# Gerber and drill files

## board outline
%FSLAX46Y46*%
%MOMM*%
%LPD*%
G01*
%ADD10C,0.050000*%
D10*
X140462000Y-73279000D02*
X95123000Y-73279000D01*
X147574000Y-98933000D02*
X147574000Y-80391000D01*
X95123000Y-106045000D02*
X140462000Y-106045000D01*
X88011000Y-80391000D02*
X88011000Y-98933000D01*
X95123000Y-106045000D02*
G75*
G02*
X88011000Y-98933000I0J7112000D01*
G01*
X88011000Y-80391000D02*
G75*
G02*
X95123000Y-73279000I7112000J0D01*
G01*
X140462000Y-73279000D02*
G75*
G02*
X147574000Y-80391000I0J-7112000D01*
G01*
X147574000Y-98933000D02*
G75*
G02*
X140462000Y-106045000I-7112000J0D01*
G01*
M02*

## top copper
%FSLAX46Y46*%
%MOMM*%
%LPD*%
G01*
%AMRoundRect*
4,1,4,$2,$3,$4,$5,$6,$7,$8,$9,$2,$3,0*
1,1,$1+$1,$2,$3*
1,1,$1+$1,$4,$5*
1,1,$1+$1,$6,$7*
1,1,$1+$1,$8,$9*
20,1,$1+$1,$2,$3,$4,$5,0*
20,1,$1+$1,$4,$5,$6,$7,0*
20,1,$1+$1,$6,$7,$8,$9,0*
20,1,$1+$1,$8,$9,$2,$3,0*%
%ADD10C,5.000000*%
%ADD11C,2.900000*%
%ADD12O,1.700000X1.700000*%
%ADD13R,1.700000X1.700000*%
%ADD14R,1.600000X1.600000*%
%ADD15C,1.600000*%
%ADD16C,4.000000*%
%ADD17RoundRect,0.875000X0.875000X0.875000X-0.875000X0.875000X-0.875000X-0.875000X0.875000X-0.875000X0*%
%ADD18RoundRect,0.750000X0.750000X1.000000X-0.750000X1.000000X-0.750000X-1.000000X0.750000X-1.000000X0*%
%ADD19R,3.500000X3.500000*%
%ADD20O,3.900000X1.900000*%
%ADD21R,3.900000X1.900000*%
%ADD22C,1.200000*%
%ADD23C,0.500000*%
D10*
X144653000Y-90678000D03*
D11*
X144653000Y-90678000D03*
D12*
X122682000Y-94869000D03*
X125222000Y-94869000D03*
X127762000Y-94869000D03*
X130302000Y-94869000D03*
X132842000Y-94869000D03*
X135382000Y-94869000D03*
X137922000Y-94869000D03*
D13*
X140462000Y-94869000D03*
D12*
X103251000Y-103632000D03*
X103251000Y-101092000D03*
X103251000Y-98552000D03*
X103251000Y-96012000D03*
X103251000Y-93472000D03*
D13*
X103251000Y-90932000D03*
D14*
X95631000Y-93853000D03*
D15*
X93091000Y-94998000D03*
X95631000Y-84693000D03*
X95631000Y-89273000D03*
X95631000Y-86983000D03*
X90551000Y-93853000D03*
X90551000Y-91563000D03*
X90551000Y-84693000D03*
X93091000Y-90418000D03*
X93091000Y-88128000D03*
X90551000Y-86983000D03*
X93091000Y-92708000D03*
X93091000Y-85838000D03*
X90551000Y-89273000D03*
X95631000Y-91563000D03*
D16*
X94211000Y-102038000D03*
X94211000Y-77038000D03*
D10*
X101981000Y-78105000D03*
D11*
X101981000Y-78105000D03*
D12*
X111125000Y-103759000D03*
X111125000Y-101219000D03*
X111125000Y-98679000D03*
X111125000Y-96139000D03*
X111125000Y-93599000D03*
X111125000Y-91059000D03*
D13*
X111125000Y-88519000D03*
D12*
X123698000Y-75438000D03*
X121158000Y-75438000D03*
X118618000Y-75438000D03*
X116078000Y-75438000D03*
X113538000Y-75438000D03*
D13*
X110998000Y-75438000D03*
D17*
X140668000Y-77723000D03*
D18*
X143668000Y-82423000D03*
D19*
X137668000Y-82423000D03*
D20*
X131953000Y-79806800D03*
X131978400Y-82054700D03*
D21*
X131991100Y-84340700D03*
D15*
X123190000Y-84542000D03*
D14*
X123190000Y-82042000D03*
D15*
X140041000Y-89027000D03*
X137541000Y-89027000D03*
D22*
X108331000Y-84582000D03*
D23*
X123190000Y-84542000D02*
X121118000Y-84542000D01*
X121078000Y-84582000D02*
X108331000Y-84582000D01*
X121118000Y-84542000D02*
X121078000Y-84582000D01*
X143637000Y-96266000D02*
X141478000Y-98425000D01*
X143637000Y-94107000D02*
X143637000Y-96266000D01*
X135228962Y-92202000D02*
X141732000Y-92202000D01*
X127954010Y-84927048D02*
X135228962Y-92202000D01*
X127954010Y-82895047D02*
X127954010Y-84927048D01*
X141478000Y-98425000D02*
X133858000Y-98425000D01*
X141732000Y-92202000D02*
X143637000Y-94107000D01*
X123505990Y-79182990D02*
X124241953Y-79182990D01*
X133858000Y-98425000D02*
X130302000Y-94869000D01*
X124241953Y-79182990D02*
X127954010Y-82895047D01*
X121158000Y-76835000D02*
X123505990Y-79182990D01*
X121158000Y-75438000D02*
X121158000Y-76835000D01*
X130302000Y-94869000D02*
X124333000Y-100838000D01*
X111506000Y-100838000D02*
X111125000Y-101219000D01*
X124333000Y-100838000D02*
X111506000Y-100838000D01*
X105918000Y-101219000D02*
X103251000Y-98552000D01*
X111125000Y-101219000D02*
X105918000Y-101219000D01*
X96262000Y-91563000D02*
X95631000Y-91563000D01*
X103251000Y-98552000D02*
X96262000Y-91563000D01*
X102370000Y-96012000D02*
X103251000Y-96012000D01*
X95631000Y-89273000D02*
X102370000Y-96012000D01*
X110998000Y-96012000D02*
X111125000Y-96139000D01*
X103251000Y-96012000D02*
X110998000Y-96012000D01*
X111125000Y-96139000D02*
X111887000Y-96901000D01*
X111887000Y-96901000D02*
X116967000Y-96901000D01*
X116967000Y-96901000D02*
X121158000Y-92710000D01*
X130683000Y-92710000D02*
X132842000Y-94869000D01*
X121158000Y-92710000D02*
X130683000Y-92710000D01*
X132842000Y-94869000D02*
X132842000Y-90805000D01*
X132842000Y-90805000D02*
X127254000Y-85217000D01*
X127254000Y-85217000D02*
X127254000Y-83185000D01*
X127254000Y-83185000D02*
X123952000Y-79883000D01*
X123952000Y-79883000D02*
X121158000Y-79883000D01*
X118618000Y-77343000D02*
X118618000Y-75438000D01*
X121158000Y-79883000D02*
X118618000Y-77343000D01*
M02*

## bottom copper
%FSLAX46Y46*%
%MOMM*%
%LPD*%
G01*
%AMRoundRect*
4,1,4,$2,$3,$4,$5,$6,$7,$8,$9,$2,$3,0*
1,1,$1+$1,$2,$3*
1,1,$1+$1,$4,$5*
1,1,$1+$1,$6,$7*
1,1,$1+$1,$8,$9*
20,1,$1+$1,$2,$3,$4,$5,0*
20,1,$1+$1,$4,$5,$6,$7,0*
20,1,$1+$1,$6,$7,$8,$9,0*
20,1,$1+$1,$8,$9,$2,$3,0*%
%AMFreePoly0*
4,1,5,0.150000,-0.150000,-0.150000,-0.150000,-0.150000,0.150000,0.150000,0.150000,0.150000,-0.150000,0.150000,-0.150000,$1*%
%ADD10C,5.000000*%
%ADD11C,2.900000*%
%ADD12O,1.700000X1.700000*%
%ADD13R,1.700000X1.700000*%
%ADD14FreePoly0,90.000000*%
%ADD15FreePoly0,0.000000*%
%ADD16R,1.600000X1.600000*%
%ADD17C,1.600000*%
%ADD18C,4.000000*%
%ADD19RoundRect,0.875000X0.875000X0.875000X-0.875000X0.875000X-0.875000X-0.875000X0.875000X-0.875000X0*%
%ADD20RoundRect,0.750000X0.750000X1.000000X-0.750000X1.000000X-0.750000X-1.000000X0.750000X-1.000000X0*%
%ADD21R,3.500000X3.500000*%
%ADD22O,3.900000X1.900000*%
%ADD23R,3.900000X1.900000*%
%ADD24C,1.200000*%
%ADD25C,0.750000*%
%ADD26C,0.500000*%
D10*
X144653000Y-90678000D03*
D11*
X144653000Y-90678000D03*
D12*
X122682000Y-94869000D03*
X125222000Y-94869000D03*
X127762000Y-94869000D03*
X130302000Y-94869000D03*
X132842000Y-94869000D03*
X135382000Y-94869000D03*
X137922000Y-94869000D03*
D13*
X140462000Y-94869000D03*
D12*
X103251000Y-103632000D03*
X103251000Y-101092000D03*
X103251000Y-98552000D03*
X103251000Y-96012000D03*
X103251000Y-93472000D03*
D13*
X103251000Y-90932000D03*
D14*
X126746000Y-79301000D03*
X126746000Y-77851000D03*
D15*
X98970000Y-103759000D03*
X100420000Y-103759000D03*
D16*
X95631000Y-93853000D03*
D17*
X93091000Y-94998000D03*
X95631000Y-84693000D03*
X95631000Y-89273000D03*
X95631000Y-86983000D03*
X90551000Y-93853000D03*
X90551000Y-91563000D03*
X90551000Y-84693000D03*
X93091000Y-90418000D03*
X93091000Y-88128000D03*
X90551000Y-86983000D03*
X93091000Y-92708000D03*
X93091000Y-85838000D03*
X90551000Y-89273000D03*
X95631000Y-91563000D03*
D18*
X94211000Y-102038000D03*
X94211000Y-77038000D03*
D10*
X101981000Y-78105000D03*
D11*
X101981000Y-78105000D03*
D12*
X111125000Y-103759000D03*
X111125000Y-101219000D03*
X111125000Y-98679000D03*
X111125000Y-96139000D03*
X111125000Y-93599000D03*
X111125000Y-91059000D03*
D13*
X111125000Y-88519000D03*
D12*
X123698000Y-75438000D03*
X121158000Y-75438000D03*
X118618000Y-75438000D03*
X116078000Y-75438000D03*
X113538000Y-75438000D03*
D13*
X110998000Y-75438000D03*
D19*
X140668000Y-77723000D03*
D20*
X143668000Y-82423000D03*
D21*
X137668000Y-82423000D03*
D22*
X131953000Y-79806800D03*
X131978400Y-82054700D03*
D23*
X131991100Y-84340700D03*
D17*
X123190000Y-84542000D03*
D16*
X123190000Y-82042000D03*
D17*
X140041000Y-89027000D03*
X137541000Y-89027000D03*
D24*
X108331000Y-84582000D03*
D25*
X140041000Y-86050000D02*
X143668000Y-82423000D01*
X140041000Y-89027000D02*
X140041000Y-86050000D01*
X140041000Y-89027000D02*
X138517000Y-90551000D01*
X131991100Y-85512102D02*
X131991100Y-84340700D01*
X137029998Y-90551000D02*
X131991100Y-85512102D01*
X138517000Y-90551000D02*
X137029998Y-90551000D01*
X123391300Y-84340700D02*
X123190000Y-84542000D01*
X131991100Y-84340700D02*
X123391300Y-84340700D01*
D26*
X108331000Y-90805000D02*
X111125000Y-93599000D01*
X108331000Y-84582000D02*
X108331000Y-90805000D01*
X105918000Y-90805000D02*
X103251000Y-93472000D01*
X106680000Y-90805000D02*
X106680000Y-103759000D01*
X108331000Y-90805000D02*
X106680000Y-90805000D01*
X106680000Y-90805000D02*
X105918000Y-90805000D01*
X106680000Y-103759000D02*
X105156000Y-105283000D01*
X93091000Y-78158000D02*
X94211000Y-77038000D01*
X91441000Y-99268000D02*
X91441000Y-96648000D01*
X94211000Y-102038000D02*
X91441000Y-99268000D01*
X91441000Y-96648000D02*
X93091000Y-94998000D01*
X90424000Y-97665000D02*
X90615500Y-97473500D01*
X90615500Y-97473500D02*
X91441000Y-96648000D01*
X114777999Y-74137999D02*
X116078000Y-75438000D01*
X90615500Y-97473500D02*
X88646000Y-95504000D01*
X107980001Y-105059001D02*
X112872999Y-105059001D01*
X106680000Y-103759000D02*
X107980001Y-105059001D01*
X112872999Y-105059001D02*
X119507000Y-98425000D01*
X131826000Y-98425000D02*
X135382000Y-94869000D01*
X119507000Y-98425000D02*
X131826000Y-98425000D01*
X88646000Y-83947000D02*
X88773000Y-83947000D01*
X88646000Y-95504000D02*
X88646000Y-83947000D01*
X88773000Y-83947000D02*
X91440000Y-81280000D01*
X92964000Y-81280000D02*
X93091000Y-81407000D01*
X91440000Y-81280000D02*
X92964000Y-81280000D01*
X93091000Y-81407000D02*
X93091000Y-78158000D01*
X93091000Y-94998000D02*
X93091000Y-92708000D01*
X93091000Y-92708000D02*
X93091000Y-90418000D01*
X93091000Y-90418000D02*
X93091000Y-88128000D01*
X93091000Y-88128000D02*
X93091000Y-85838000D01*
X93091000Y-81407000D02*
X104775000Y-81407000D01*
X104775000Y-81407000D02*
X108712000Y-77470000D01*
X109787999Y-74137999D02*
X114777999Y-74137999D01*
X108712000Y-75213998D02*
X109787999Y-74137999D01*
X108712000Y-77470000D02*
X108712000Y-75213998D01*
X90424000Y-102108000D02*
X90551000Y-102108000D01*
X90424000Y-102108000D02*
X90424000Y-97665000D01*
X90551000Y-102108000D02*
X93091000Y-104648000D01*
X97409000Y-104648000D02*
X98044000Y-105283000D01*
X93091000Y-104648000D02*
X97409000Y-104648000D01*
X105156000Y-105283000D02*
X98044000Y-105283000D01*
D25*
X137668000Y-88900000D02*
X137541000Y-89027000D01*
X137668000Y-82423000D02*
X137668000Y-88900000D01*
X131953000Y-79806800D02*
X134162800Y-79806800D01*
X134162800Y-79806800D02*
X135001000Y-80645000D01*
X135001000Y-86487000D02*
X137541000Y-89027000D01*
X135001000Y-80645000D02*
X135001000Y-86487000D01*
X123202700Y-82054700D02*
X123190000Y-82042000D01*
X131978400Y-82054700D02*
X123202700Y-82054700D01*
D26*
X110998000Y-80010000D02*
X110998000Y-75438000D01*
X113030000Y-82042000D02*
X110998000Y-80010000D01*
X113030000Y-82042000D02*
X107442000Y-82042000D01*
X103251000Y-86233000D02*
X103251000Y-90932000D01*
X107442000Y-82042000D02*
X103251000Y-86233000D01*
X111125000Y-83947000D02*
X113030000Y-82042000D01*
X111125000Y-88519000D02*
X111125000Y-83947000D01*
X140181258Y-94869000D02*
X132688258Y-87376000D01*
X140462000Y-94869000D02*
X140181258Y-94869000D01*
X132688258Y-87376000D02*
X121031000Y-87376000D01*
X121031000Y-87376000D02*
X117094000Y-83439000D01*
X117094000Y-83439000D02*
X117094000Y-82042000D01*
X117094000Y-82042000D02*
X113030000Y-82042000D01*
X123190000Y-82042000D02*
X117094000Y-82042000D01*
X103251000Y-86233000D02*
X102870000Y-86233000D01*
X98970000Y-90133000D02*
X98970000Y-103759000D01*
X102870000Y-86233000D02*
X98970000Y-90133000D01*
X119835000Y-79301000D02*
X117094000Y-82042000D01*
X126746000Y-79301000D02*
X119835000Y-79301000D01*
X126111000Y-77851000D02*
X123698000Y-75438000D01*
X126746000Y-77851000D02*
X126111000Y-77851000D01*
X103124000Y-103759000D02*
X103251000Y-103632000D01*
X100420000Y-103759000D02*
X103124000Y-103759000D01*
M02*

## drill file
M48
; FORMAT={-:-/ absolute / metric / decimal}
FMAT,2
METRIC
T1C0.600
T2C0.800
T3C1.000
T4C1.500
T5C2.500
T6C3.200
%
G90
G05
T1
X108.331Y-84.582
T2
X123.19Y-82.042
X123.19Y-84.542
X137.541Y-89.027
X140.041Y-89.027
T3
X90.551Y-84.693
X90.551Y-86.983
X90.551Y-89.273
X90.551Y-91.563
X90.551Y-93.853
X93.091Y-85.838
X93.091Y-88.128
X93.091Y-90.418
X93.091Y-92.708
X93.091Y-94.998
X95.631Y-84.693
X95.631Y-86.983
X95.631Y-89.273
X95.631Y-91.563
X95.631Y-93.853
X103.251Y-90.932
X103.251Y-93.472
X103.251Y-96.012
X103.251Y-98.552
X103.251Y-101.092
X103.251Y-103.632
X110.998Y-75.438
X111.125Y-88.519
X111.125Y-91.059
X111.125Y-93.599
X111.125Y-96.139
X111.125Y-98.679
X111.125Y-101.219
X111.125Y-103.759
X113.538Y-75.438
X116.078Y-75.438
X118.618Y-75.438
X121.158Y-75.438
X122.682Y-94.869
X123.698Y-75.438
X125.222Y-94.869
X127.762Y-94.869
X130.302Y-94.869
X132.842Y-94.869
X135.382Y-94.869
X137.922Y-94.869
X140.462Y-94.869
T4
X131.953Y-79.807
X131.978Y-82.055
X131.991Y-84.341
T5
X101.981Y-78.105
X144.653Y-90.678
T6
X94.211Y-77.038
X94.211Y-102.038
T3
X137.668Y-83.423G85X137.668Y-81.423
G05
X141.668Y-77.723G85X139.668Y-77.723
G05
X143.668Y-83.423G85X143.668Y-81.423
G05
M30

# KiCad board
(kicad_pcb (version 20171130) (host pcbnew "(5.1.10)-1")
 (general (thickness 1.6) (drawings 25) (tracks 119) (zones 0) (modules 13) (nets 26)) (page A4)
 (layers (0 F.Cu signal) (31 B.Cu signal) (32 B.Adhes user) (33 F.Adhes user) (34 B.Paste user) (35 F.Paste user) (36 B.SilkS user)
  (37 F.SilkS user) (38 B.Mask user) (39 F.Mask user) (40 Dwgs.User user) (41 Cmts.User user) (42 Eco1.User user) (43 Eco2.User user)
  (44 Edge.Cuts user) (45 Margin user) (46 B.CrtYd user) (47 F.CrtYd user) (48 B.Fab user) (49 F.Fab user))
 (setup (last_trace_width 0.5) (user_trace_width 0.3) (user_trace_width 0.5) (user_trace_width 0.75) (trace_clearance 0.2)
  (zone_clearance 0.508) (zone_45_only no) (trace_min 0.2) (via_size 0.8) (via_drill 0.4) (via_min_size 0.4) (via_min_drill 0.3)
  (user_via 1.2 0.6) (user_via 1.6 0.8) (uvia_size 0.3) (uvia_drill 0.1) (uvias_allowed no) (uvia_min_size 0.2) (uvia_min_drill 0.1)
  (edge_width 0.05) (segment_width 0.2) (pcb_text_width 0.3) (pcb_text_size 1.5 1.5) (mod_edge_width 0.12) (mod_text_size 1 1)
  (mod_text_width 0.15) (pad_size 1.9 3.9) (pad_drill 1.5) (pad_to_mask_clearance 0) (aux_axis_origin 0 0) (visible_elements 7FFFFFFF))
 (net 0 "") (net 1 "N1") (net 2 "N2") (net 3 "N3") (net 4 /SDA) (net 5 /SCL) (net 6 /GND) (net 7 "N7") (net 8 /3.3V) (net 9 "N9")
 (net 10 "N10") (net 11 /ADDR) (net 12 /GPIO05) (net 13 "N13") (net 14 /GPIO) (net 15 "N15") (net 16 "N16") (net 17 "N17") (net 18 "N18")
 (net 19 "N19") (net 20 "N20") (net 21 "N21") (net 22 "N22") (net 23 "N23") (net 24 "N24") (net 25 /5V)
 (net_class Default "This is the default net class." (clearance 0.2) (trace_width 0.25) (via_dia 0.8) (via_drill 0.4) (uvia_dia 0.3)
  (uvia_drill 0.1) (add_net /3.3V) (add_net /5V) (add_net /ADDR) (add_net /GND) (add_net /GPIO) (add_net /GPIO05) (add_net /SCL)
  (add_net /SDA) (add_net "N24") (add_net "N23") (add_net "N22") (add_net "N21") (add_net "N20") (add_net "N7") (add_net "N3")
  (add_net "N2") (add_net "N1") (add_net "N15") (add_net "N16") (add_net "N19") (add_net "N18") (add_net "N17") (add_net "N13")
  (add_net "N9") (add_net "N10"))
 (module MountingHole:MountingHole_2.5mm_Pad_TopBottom (layer F.Cu) (at 144.653 90.678)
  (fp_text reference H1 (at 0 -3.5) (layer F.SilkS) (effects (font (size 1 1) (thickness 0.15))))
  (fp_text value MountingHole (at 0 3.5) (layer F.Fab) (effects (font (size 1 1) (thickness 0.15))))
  (pad 1 connect circle (at 0 0) (size 5 5) (layers B.Cu B.Mask))
  (pad 1 connect circle (at 0 0) (size 5 5) (layers F.Cu F.Mask))
  (pad 1 thru_hole circle (at 0 0) (size 2.9 2.9) (drill 2.5) (layers *.Cu *.Mask)))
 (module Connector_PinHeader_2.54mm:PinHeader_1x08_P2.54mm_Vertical (layer F.Cu) (at 140.462 94.869 270)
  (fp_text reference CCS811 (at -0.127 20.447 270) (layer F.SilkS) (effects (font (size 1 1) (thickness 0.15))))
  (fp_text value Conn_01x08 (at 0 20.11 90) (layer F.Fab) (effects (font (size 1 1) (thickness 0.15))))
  (pad 8 thru_hole oval (at 0 17.78 270) (size 1.7 1.7) (drill 1) (layers *.Cu *.Mask) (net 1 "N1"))
  (pad 7 thru_hole oval (at 0 15.24 270) (size 1.7 1.7) (drill 1) (layers *.Cu *.Mask) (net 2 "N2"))
  (pad 6 thru_hole oval (at 0 12.7 270) (size 1.7 1.7) (drill 1) (layers *.Cu *.Mask) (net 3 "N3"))
  (pad 5 thru_hole oval (at 0 10.16 270) (size 1.7 1.7) (drill 1) (layers *.Cu *.Mask) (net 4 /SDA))
  (pad 4 thru_hole oval (at 0 7.62 270) (size 1.7 1.7) (drill 1) (layers *.Cu *.Mask) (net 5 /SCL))
  (pad 3 thru_hole oval (at 0 5.08 270) (size 1.7 1.7) (drill 1) (layers *.Cu *.Mask) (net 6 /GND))
  (pad 2 thru_hole oval (at 0 2.54 270) (size 1.7 1.7) (drill 1) (layers *.Cu *.Mask) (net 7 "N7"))
  (pad 1 thru_hole rect (at 0 0 270) (size 1.7 1.7) (drill 1) (layers *.Cu *.Mask) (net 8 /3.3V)))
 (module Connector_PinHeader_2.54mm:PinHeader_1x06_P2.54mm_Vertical (layer F.Cu) (at 103.251 90.932)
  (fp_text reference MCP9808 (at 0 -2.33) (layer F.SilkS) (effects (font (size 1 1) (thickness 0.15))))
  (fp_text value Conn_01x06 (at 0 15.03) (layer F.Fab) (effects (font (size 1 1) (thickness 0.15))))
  (pad 6 thru_hole oval (at 0 12.7) (size 1.7 1.7) (drill 1) (layers *.Cu *.Mask) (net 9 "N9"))
  (pad 5 thru_hole oval (at 0 10.16) (size 1.7 1.7) (drill 1) (layers *.Cu *.Mask) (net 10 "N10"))
  (pad 4 thru_hole oval (at 0 7.62) (size 1.7 1.7) (drill 1) (layers *.Cu *.Mask) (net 4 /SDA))
  (pad 3 thru_hole oval (at 0 5.08) (size 1.7 1.7) (drill 1) (layers *.Cu *.Mask) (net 5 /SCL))
  (pad 2 thru_hole oval (at 0 2.54) (size 1.7 1.7) (drill 1) (layers *.Cu *.Mask) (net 6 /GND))
  (pad 1 thru_hole rect (at 0 0) (size 1.7 1.7) (drill 1) (layers *.Cu *.Mask) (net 8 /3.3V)))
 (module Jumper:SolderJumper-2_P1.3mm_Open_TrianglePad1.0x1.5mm (layer B.Cu) (at 126.746 78.576 90)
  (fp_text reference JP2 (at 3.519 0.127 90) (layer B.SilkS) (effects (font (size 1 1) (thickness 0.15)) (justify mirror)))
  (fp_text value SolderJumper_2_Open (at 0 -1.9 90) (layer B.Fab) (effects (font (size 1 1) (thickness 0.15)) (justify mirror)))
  (pad 1 smd custom (at -0.725 0 90) (size 0.3 0.3) (layers B.Cu B.Mask) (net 8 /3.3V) (zone_connect 2)
   (options (clearance outline) (anchor rect)) (primitives))
  (pad 2 smd custom (at 0.725 0 90) (size 0.3 0.3) (layers B.Cu B.Mask) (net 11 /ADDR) (zone_connect 2)
   (options (clearance outline) (anchor rect)) (primitives)))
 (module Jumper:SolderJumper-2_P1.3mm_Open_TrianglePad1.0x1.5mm (layer B.Cu) (at 99.695 103.759)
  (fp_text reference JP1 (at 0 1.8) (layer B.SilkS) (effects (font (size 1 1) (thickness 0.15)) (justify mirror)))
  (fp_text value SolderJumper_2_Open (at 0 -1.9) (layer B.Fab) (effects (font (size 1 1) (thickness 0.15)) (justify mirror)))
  (pad 1 smd custom (at -0.725 0) (size 0.3 0.3) (layers B.Cu B.Mask) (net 8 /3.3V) (zone_connect 2)
   (options (clearance outline) (anchor rect)) (primitives))
  (pad 2 smd custom (at 0.725 0) (size 0.3 0.3) (layers B.Cu B.Mask) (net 9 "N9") (zone_connect 2)
   (options (clearance outline) (anchor rect)) (primitives)))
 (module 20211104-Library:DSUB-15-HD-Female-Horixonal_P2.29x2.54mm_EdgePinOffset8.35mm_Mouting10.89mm (layer F.Cu) (at 95.631 93.853 270)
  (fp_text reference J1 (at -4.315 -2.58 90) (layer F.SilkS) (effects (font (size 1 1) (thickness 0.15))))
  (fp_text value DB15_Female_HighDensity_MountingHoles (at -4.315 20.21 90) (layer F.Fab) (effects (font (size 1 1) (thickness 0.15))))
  (pad 1 thru_hole rect (at 0 0 270) (size 1.6 1.6) (drill 1) (layers *.Cu *.Mask) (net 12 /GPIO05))
  (pad 6 thru_hole circle (at 1.145 2.54 270) (size 1.6 1.6) (drill 1) (layers *.Cu *.Mask) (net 6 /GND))
  (pad 5 thru_hole circle (at -9.16 0 270) (size 1.6 1.6) (drill 1) (layers *.Cu *.Mask) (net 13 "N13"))
  (pad 3 thru_hole circle (at -4.58 0 270) (size 1.6 1.6) (drill 1) (layers *.Cu *.Mask) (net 5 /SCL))
  (pad 4 thru_hole circle (at -6.87 0 270) (size 1.6 1.6) (drill 1) (layers *.Cu *.Mask) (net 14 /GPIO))
  (pad 11 thru_hole circle (at 0 5.08 270) (size 1.6 1.6) (drill 1) (layers *.Cu *.Mask) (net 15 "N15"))
  (pad 12 thru_hole circle (at -2.29 5.08 270) (size 1.6 1.6) (drill 1) (layers *.Cu *.Mask) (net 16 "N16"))
  (pad 15 thru_hole circle (at -9.16 5.08 270) (size 1.6 1.6) (drill 1) (layers *.Cu *.Mask) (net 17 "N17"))
  (pad 8 thru_hole circle (at -3.435 2.54 270) (size 1.6 1.6) (drill 1) (layers *.Cu *.Mask) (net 6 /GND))
  (pad 9 thru_hole circle (at -5.725 2.54 270) (size 1.6 1.6) (drill 1) (layers *.Cu *.Mask) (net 6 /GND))
  (pad 14 thru_hole circle (at -6.87 5.08 270) (size 1.6 1.6) (drill 1) (layers *.Cu *.Mask) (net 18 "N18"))
  (pad 7 thru_hole circle (at -1.145 2.54 270) (size 1.6 1.6) (drill 1) (layers *.Cu *.Mask) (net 6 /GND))
  (pad 10 thru_hole circle (at -8.015 2.54 270) (size 1.6 1.6) (drill 1) (layers *.Cu *.Mask) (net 6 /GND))
  (pad 13 thru_hole circle (at -4.58 5.08 270) (size 1.6 1.6) (drill 1) (layers *.Cu *.Mask) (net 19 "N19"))
  (pad 2 thru_hole circle (at -2.29 0 270) (size 1.6 1.6) (drill 1) (layers *.Cu *.Mask) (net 4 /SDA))
  (pad 0 thru_hole circle (at 8.185 1.42 270) (size 4 4) (drill 3.2) (layers *.Cu *.Mask) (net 6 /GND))
  (pad 0 thru_hole circle (at -16.815 1.42 270) (size 4 4) (drill 3.2) (layers *.Cu *.Mask) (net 6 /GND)))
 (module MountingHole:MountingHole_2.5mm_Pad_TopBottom (layer F.Cu) (at 101.981 78.105)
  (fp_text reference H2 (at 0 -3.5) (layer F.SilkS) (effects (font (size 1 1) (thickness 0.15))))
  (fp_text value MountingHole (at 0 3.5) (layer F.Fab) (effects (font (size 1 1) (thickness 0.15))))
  (pad 1 connect circle (at 0 0) (size 5 5) (layers B.Cu B.Mask))
  (pad 1 connect circle (at 0 0) (size 5 5) (layers F.Cu F.Mask))
  (pad 1 thru_hole circle (at 0 0) (size 2.9 2.9) (drill 2.5) (layers *.Cu *.Mask)))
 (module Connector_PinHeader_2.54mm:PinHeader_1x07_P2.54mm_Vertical (layer F.Cu) (at 111.125 88.519)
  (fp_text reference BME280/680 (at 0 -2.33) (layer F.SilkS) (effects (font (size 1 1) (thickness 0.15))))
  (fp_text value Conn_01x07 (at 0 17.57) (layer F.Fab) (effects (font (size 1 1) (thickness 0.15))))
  (pad 7 thru_hole oval (at 0 15.24) (size 1.7 1.7) (drill 1) (layers *.Cu *.Mask) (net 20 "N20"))
  (pad 6 thru_hole oval (at 0 12.7) (size 1.7 1.7) (drill 1) (layers *.Cu *.Mask) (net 4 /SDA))
  (pad 5 thru_hole oval (at 0 10.16) (size 1.7 1.7) (drill 1) (layers *.Cu *.Mask) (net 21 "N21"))
  (pad 4 thru_hole oval (at 0 7.62) (size 1.7 1.7) (drill 1) (layers *.Cu *.Mask) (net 5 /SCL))
  (pad 3 thru_hole oval (at 0 5.08) (size 1.7 1.7) (drill 1) (layers *.Cu *.Mask) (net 6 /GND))
  (pad 2 thru_hole oval (at 0 2.54) (size 1.7 1.7) (drill 1) (layers *.Cu *.Mask) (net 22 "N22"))
  (pad 1 thru_hole rect (at 0 0) (size 1.7 1.7) (drill 1) (layers *.Cu *.Mask) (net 8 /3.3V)))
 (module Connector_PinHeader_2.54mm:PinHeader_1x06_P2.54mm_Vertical (layer F.Cu) (at 110.998 75.438 90)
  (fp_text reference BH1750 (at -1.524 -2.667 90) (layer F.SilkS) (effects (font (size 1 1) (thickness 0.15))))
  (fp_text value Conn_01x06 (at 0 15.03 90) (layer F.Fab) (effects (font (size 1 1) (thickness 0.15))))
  (pad 6 thru_hole oval (at 0 12.7 90) (size 1.7 1.7) (drill 1) (layers *.Cu *.Mask) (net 11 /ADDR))
  (pad 5 thru_hole oval (at 0 10.16 90) (size 1.7 1.7) (drill 1) (layers *.Cu *.Mask) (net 4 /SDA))
  (pad 4 thru_hole oval (at 0 7.62 90) (size 1.7 1.7) (drill 1) (layers *.Cu *.Mask) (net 5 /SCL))
  (pad 3 thru_hole oval (at 0 5.08 90) (size 1.7 1.7) (drill 1) (layers *.Cu *.Mask) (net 6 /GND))
  (pad 2 thru_hole oval (at 0 2.54 90) (size 1.7 1.7) (drill 1) (layers *.Cu *.Mask) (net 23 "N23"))
  (pad 1 thru_hole rect (at 0 0 90) (size 1.7 1.7) (drill 1) (layers *.Cu *.Mask) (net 8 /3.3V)))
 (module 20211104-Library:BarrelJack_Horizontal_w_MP (layer F.Cu) (at 137.668 82.423 180)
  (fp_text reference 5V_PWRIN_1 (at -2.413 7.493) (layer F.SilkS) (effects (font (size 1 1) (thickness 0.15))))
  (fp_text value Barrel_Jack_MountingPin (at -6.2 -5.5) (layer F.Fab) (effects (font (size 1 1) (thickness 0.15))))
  (pad MP thru_hole roundrect (at -3 4.7 180) (size 3.5 3.5) (drill oval 3 1) (layers *.Cu *.Mask) (roundrect_rratio 0.25) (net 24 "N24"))
  (pad 2 thru_hole roundrect (at -6 0 180) (size 3 3.5) (drill oval 1 3) (layers *.Cu *.Mask) (roundrect_rratio 0.25) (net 6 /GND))
  (pad 1 thru_hole rect (at 0 0 180) (size 3.5 3.5) (drill oval 1 3) (layers *.Cu *.Mask) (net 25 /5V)))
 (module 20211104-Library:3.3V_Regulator (layer F.Cu) (at 131.953 87.503 90)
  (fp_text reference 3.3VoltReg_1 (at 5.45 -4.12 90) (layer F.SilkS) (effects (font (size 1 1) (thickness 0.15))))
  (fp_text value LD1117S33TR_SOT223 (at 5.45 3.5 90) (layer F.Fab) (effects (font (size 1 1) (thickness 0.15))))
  (pad 3 thru_hole oval (at 7.6962 0 90) (size 1.9 3.9) (drill 1.5) (layers *.Cu *.Mask) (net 25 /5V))
  (pad 2 thru_hole oval (at 5.4483 0.0254 90) (size 1.9 3.9) (drill 1.5) (layers *.Cu *.Mask) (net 8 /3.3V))
  (pad 1 thru_hole rect (at 3.1623 0.0381 90) (size 1.9 3.9) (drill 1.5) (layers *.Cu *.Mask) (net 6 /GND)))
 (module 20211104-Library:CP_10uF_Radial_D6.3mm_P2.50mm (layer F.Cu) (at 123.19 82.042 270)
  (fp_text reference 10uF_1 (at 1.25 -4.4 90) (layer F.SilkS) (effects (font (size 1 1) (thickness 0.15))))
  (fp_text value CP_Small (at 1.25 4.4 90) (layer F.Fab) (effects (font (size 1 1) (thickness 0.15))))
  (pad 2 thru_hole circle (at 2.5 0 270) (size 1.6 1.6) (drill 0.8) (layers *.Cu *.Mask) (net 6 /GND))
  (pad 1 thru_hole rect (at 0 0 270) (size 1.6 1.6) (drill 0.8) (layers *.Cu *.Mask) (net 8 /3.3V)))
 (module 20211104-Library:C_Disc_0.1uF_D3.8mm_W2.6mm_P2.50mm (layer F.Cu) (at 137.541 89.027)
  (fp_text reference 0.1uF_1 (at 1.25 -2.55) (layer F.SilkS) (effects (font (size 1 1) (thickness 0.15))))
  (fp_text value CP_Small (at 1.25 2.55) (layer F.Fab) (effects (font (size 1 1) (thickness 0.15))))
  (pad 2 thru_hole circle (at 2.5 0) (size 1.6 1.6) (drill 0.8) (layers *.Cu *.Mask) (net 6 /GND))
  (pad 1 thru_hole circle (at 0 0) (size 1.6 1.6) (drill 0.8) (layers *.Cu *.Mask) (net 25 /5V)))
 (gr_line (start 140.462 73.279) (end 95.123 73.279) (layer Edge.Cuts) (width 0.05))
 (gr_line (start 147.574 98.933) (end 147.574 80.391) (layer Edge.Cuts) (width 0.05))
 (gr_line (start 95.123 106.045) (end 140.462 106.045) (layer Edge.Cuts) (width 0.05))
 (gr_line (start 88.011 80.391) (end 88.011 98.933) (layer Edge.Cuts) (width 0.05))
 (gr_arc (start 95.123 98.933) (end 88.011 98.933) (angle -90) (layer Edge.Cuts) (width 0.05))
 (gr_arc (start 95.123 80.391) (end 95.123 73.279) (angle -90) (layer Edge.Cuts) (width 0.05))
 (gr_arc (start 140.462 80.391) (end 147.574 80.391) (angle -90) (layer Edge.Cuts) (width 0.05))
 (gr_arc (start 140.462 98.933) (end 140.462 106.045) (angle -90) (layer Edge.Cuts) (width 0.05))
 (segment (start 140.041 86.05) (end 143.668 82.423) (width 0.75) (layer B.Cu) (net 6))
 (segment (start 140.041 89.027) (end 140.041 86.05) (width 0.75) (layer B.Cu) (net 6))
 (segment (start 140.041 89.027) (end 138.517 90.551) (width 0.75) (layer B.Cu) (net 6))
 (segment (start 131.9911 85.512102) (end 131.9911 84.3407) (width 0.75) (layer B.Cu) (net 6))
 (segment (start 137.029998 90.551) (end 131.9911 85.512102) (width 0.75) (layer B.Cu) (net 6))
 (segment (start 138.517 90.551) (end 137.029998 90.551) (width 0.75) (layer B.Cu) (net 6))
 (segment (start 123.3913 84.3407) (end 123.19 84.542) (width 0.75) (layer B.Cu) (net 6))
 (segment (start 131.9911 84.3407) (end 123.3913 84.3407) (width 0.75) (layer B.Cu) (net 6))
 (segment (start 123.19 84.542) (end 121.118 84.542) (width 0.5) (layer F.Cu) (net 6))
 (via (at 108.331 84.582) (size 1.2) (drill 0.6) (layers F.Cu B.Cu) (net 6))
 (segment (start 121.078 84.582) (end 108.331 84.582) (width 0.5) (layer F.Cu) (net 6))
 (segment (start 121.118 84.542) (end 121.078 84.582) (width 0.5) (layer F.Cu) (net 6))
 (segment (start 108.331 90.805) (end 111.125 93.599) (width 0.5) (layer B.Cu) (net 6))
 (segment (start 108.331 84.582) (end 108.331 90.805) (width 0.5) (layer B.Cu) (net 6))
 (segment (start 105.918 90.805) (end 103.251 93.472) (width 0.5) (layer B.Cu) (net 6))
 (segment (start 106.68 90.805) (end 106.68 103.759) (width 0.5) (layer B.Cu) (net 6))
 (segment (start 108.331 90.805) (end 106.68 90.805) (width 0.5) (layer B.Cu) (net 6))
 (segment (start 106.68 90.805) (end 105.918 90.805) (width 0.5) (layer B.Cu) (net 6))
 (segment (start 106.68 103.759) (end 105.156 105.283) (width 0.5) (layer B.Cu) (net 6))
 (segment (start 93.091 78.158) (end 94.211 77.038) (width 0.5) (layer B.Cu) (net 6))
 (segment (start 91.441 99.268) (end 91.441 96.648) (width 0.5) (layer B.Cu) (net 6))
 (segment (start 94.211 102.038) (end 91.441 99.268) (width 0.5) (layer B.Cu) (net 6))
 (segment (start 91.441 96.648) (end 93.091 94.998) (width 0.5) (layer B.Cu) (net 6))
 (segment (start 90.424 97.665) (end 90.6155 97.4735) (width 0.5) (layer B.Cu) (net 6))
 (segment (start 90.6155 97.4735) (end 91.441 96.648) (width 0.5) (layer B.Cu) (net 6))
 (segment (start 114.777999 74.137999) (end 116.078 75.438) (width 0.5) (layer B.Cu) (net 6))
 (segment (start 90.6155 97.4735) (end 88.646 95.504) (width 0.5) (layer B.Cu) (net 6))
 (segment (start 107.980001 105.059001) (end 112.872999 105.059001) (width 0.5) (layer B.Cu) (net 6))
 (segment (start 106.68 103.759) (end 107.980001 105.059001) (width 0.5) (layer B.Cu) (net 6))
 (segment (start 112.872999 105.059001) (end 119.507 98.425) (width 0.5) (layer B.Cu) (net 6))
 (segment (start 131.826 98.425) (end 135.382 94.869) (width 0.5) (layer B.Cu) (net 6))
 (segment (start 119.507 98.425) (end 131.826 98.425) (width 0.5) (layer B.Cu) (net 6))
 (segment (start 88.646 83.947) (end 88.773 83.947) (width 0.5) (layer B.Cu) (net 6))
 (segment (start 88.646 95.504) (end 88.646 83.947) (width 0.5) (layer B.Cu) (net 6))
 (segment (start 88.773 83.947) (end 91.44 81.28) (width 0.5) (layer B.Cu) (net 6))
 (segment (start 92.964 81.28) (end 93.091 81.407) (width 0.5) (layer B.Cu) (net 6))
 (segment (start 91.44 81.28) (end 92.964 81.28) (width 0.5) (layer B.Cu) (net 6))
 (segment (start 93.091 81.407) (end 93.091 78.158) (width 0.5) (layer B.Cu) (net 6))
 (segment (start 93.091 94.998) (end 93.091 92.708) (width 0.5) (layer B.Cu) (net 6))
 (segment (start 93.091 92.708) (end 93.091 90.418) (width 0.5) (layer B.Cu) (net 6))
 (segment (start 93.091 90.418) (end 93.091 88.128) (width 0.5) (layer B.Cu) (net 6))
 (segment (start 93.091 88.128) (end 93.091 85.838) (width 0.5) (layer B.Cu) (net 6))
 (segment (start 93.091 81.407) (end 104.775 81.407) (width 0.5) (layer B.Cu) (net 6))
 (segment (start 104.775 81.407) (end 108.712 77.47) (width 0.5) (layer B.Cu) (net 6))
 (segment (start 109.787999 74.137999) (end 114.777999 74.137999) (width 0.5) (layer B.Cu) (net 6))
 (segment (start 108.712 75.213998) (end 109.787999 74.137999) (width 0.5) (layer B.Cu) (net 6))
 (segment (start 108.712 77.47) (end 108.712 75.213998) (width 0.5) (layer B.Cu) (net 6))
 (segment (start 90.424 102.108) (end 90.551 102.108) (width 0.5) (layer B.Cu) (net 6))
 (segment (start 90.424 102.108) (end 90.424 97.665) (width 0.5) (layer B.Cu) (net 6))
 (segment (start 90.551 102.108) (end 93.091 104.648) (width 0.5) (layer B.Cu) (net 6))
 (segment (start 97.409 104.648) (end 98.044 105.283) (width 0.5) (layer B.Cu) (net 6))
 (segment (start 93.091 104.648) (end 97.409 104.648) (width 0.5) (layer B.Cu) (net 6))
 (segment (start 105.156 105.283) (end 98.044 105.283) (width 0.5) (layer B.Cu) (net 6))
 (segment (start 137.668 88.9) (end 137.541 89.027) (width 0.75) (layer B.Cu) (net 25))
 (segment (start 137.668 82.423) (end 137.668 88.9) (width 0.75) (layer B.Cu) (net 25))
 (segment (start 131.953 79.8068) (end 134.1628 79.8068) (width 0.75) (layer B.Cu) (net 25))
 (segment (start 134.1628 79.8068) (end 135.001 80.645) (width 0.75) (layer B.Cu) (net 25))
 (segment (start 135.001 86.487) (end 137.541 89.027) (width 0.75) (layer B.Cu) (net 25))
 (segment (start 135.001 80.645) (end 135.001 86.487) (width 0.75) (layer B.Cu) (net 25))
 (segment (start 123.2027 82.0547) (end 123.19 82.042) (width 0.75) (layer B.Cu) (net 8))
 (segment (start 131.9784 82.0547) (end 123.2027 82.0547) (width 0.75) (layer B.Cu) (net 8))
 (segment (start 110.998 80.01) (end 110.998 75.438) (width 0.5) (layer B.Cu) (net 8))
 (segment (start 113.03 82.042) (end 110.998 80.01) (width 0.5) (layer B.Cu) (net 8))
 (segment (start 113.03 82.042) (end 107.442 82.042) (width 0.5) (layer B.Cu) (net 8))
 (segment (start 103.251 86.233) (end 103.251 90.932) (width 0.5) (layer B.Cu) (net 8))
 (segment (start 107.442 82.042) (end 103.251 86.233) (width 0.5) (layer B.Cu) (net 8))
 (segment (start 111.125 83.947) (end 113.03 82.042) (width 0.5) (layer B.Cu) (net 8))
 (segment (start 111.125 88.519) (end 111.125 83.947) (width 0.5) (layer B.Cu) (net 8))
 (segment (start 140.181258 94.869) (end 132.688258 87.376) (width 0.5) (layer B.Cu) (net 8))
 (segment (start 140.462 94.869) (end 140.181258 94.869) (width 0.5) (layer B.Cu) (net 8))
 (segment (start 132.688258 87.376) (end 121.031 87.376) (width 0.5) (layer B.Cu) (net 8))
 (segment (start 121.031 87.376) (end 117.094 83.439) (width 0.5) (layer B.Cu) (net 8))
 (segment (start 117.094 83.439) (end 117.094 82.042) (width 0.5) (layer B.Cu) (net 8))
 (segment (start 117.094 82.042) (end 113.03 82.042) (width 0.5) (layer B.Cu) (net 8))
 (segment (start 123.19 82.042) (end 117.094 82.042) (width 0.5) (layer B.Cu) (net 8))
 (segment (start 103.251 86.233) (end 102.87 86.233) (width 0.5) (layer B.Cu) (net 8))
 (segment (start 98.97 90.133) (end 98.97 103.759) (width 0.5) (layer B.Cu) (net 8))
 (segment (start 102.87 86.233) (end 98.97 90.133) (width 0.5) (layer B.Cu) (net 8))
 (segment (start 119.835 79.301) (end 117.094 82.042) (width 0.5) (layer B.Cu) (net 8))
 (segment (start 126.746 79.301) (end 119.835 79.301) (width 0.5) (layer B.Cu) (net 8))
 (segment (start 126.111 77.851) (end 123.698 75.438) (width 0.5) (layer B.Cu) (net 11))
 (segment (start 126.746 77.851) (end 126.111 77.851) (width 0.5) (layer B.Cu) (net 11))
 (segment (start 143.637 96.266) (end 141.478 98.425) (width 0.5) (layer F.Cu) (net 4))
 (segment (start 143.637 94.107) (end 143.637 96.266) (width 0.5) (layer F.Cu) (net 4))
 (segment (start 135.228962 92.202) (end 141.732 92.202) (width 0.5) (layer F.Cu) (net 4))
 (segment (start 127.95401 84.927048) (end 135.228962 92.202) (width 0.5) (layer F.Cu) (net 4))
 (segment (start 127.95401 82.895047) (end 127.95401 84.927048) (width 0.5) (layer F.Cu) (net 4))
 (segment (start 141.478 98.425) (end 133.858 98.425) (width 0.5) (layer F.Cu) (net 4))
 (segment (start 141.732 92.202) (end 143.637 94.107) (width 0.5) (layer F.Cu) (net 4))
 (segment (start 123.50599 79.18299) (end 124.241953 79.18299) (width 0.5) (layer F.Cu) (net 4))
 (segment (start 133.858 98.425) (end 130.302 94.869) (width 0.5) (layer F.Cu) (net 4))
 (segment (start 124.241953 79.18299) (end 127.95401 82.895047) (width 0.5) (layer F.Cu) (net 4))
 (segment (start 121.158 76.835) (end 123.50599 79.18299) (width 0.5) (layer F.Cu) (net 4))
 (segment (start 121.158 75.438) (end 121.158 76.835) (width 0.5) (layer F.Cu) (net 4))
 (segment (start 130.302 94.869) (end 124.333 100.838) (width 0.5) (layer F.Cu) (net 4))
 (segment (start 111.506 100.838) (end 111.125 101.219) (width 0.5) (layer F.Cu) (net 4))
 (segment (start 124.333 100.838) (end 111.506 100.838) (width 0.5) (layer F.Cu) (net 4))
 (segment (start 105.918 101.219) (end 103.251 98.552) (width 0.5) (layer F.Cu) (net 4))
 (segment (start 111.125 101.219) (end 105.918 101.219) (width 0.5) (layer F.Cu) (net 4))
 (segment (start 96.262 91.563) (end 95.631 91.563) (width 0.5) (layer F.Cu) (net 4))
 (segment (start 103.251 98.552) (end 96.262 91.563) (width 0.5) (layer F.Cu) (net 4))
 (segment (start 102.37 96.012) (end 103.251 96.012) (width 0.5) (layer F.Cu) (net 5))
 (segment (start 95.631 89.273) (end 102.37 96.012) (width 0.5) (layer F.Cu) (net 5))
 (segment (start 110.998 96.012) (end 111.125 96.139) (width 0.5) (layer F.Cu) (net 5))
 (segment (start 103.251 96.012) (end 110.998 96.012) (width 0.5) (layer F.Cu) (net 5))
 (segment (start 111.125 96.139) (end 111.887 96.901) (width 0.5) (layer F.Cu) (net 5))
 (segment (start 111.887 96.901) (end 116.967 96.901) (width 0.5) (layer F.Cu) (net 5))
 (segment (start 116.967 96.901) (end 121.158 92.71) (width 0.5) (layer F.Cu) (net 5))
 (segment (start 130.683 92.71) (end 132.842 94.869) (width 0.5) (layer F.Cu) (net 5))
 (segment (start 121.158 92.71) (end 130.683 92.71) (width 0.5) (layer F.Cu) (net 5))
 (segment (start 132.842 94.869) (end 132.842 90.805) (width 0.5) (layer F.Cu) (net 5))
 (segment (start 132.842 90.805) (end 127.254 85.217) (width 0.5) (layer F.Cu) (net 5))
 (segment (start 127.254 85.217) (end 127.254 83.185) (width 0.5) (layer F.Cu) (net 5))
 (segment (start 127.254 83.185) (end 123.952 79.883) (width 0.5) (layer F.Cu) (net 5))
 (segment (start 123.952 79.883) (end 121.158 79.883) (width 0.5) (layer F.Cu) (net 5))
 (segment (start 118.618 77.343) (end 118.618 75.438) (width 0.5) (layer F.Cu) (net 5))
 (segment (start 121.158 79.883) (end 118.618 77.343) (width 0.5) (layer F.Cu) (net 5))
 (segment (start 103.124 103.759) (end 103.251 103.632) (width 0.5) (layer B.Cu) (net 9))
 (segment (start 100.42 103.759) (end 103.124 103.759) (width 0.5) (layer B.Cu) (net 9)))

